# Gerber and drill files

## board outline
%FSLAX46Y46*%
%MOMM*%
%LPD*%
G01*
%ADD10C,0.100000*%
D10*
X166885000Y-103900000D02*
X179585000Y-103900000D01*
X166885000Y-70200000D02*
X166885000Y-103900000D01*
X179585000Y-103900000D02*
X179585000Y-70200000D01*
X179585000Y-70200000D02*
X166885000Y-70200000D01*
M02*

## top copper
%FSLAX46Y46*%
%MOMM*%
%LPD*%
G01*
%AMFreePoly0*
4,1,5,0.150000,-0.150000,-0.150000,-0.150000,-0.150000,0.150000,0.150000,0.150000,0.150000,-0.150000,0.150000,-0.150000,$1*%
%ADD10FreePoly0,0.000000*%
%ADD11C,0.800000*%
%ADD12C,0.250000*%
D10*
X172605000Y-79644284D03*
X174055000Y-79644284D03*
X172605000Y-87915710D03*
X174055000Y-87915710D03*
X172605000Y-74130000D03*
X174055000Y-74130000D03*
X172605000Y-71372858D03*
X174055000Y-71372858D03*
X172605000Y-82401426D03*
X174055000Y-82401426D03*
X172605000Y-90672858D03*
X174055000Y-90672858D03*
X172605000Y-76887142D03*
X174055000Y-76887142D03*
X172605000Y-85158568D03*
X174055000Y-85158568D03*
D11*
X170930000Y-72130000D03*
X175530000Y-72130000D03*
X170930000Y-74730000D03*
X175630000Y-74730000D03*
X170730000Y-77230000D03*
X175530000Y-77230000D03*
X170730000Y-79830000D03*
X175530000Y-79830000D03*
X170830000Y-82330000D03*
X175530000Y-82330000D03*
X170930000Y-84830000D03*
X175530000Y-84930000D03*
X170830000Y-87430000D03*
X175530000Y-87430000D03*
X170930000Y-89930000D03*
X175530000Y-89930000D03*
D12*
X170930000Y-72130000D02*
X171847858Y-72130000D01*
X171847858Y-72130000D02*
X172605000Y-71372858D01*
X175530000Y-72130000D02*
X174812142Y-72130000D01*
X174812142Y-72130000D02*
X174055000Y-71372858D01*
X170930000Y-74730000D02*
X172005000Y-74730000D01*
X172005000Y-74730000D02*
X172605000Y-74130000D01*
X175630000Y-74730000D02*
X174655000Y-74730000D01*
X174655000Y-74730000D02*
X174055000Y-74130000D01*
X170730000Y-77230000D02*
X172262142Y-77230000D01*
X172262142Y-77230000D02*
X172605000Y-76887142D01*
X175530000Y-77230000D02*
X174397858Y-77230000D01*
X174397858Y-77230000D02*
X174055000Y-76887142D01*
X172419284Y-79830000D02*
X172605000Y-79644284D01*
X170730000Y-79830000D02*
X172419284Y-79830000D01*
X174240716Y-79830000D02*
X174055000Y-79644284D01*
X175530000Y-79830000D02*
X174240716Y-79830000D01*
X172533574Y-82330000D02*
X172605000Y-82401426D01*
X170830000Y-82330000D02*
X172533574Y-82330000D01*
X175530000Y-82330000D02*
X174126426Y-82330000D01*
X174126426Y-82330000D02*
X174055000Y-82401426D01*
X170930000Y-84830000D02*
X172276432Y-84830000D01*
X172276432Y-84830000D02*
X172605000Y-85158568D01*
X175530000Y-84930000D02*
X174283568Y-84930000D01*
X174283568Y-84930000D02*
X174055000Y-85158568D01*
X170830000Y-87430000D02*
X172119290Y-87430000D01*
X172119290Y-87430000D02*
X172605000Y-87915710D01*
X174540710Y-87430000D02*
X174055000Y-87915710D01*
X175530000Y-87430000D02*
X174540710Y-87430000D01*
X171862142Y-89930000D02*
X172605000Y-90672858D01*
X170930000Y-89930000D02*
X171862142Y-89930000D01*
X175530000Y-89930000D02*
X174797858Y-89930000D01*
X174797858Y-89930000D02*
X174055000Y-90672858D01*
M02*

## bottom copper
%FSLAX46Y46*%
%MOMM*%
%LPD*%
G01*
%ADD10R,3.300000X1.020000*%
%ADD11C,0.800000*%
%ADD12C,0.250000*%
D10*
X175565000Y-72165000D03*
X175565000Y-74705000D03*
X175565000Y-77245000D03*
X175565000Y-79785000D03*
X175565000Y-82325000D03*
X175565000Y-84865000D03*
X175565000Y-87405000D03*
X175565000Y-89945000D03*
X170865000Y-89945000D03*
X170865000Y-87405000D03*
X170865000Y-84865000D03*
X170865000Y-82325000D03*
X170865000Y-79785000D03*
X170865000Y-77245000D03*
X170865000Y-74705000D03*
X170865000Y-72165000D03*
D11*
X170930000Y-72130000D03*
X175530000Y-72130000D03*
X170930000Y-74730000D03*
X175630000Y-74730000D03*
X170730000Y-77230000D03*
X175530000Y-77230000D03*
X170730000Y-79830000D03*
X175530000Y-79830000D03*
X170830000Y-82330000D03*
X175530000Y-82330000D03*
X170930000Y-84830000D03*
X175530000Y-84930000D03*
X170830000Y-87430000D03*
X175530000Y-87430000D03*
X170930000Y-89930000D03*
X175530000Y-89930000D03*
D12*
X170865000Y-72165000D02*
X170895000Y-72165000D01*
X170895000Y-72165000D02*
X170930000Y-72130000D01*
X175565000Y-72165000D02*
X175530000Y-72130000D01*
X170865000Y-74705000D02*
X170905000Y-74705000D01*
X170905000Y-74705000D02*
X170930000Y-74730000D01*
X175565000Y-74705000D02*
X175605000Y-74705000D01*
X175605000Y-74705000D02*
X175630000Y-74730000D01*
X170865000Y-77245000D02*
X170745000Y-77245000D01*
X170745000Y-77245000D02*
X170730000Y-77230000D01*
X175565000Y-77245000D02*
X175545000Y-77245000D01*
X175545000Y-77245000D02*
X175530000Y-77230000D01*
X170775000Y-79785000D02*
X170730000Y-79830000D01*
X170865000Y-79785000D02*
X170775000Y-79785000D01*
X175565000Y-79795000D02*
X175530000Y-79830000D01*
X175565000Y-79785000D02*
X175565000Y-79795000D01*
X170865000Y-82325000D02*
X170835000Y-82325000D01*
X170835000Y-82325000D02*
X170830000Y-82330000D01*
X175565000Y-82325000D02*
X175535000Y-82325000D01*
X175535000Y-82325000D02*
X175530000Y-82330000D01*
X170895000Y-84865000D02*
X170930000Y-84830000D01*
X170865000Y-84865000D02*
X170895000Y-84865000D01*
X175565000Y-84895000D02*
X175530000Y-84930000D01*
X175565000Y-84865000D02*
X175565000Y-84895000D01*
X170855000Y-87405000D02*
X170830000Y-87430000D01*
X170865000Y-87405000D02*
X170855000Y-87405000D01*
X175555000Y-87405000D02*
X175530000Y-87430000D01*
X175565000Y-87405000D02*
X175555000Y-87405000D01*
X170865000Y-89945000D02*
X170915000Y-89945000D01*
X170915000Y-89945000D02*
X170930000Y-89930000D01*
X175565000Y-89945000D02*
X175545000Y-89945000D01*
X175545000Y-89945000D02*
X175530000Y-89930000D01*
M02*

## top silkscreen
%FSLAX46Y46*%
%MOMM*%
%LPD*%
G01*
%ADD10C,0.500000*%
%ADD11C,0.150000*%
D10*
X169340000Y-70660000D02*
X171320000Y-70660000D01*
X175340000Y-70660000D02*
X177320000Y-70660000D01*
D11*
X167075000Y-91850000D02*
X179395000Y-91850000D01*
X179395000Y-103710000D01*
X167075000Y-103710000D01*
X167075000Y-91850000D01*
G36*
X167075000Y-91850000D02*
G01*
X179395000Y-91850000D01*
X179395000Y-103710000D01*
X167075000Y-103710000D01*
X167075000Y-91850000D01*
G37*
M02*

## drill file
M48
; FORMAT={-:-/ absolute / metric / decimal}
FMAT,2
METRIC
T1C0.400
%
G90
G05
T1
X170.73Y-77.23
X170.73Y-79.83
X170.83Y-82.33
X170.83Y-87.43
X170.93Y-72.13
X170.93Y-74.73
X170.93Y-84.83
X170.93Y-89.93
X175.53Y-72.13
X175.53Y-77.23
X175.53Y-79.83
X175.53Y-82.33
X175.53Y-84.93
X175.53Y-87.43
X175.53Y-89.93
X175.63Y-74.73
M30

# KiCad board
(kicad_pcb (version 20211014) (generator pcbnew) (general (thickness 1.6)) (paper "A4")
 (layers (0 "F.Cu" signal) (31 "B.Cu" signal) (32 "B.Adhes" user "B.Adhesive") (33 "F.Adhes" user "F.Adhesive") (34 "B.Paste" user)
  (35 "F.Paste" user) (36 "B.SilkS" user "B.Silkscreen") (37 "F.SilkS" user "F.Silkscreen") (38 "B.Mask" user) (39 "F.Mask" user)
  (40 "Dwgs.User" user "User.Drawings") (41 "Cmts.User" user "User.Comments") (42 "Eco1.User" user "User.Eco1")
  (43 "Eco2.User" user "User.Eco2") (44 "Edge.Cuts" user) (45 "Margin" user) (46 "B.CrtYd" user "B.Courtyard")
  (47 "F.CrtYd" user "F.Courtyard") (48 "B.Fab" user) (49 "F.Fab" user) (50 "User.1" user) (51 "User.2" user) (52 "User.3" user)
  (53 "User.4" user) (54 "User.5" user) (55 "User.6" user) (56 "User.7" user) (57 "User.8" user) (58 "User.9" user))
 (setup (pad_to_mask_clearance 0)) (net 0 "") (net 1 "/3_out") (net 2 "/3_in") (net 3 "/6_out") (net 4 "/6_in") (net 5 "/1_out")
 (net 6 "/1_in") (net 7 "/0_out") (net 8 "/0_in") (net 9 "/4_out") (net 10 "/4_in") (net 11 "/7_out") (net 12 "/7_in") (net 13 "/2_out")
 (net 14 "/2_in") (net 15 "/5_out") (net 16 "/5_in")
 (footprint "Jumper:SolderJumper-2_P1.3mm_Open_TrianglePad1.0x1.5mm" (layer "F.Cu") (at 173.33 79.644284)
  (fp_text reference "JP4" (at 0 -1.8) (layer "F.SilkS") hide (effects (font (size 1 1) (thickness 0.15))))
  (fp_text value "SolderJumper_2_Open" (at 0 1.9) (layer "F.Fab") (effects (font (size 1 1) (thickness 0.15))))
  (pad "1" smd custom (at -0.725 0) (size 0.3 0.3) (layers "F.Cu" "F.Mask") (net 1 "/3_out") (zone_connect 2)
   (options (clearance outline) (anchor rect)) (primitives))
  (pad "2" smd custom (at 0.725 0) (size 0.3 0.3) (layers "F.Cu" "F.Mask") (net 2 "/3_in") (zone_connect 2)
   (options (clearance outline) (anchor rect)) (primitives)))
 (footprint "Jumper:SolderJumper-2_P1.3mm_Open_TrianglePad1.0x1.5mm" (layer "F.Cu") (at 173.33 87.91571)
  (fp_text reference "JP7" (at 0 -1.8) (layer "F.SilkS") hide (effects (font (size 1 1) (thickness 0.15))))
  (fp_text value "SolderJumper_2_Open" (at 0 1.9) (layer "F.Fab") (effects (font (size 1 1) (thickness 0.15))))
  (pad "1" smd custom (at -0.725 0) (size 0.3 0.3) (layers "F.Cu" "F.Mask") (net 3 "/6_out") (zone_connect 2)
   (options (clearance outline) (anchor rect)) (primitives))
  (pad "2" smd custom (at 0.725 0) (size 0.3 0.3) (layers "F.Cu" "F.Mask") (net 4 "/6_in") (zone_connect 2)
   (options (clearance outline) (anchor rect)) (primitives)))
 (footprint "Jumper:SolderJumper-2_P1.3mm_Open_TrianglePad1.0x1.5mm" (layer "F.Cu") (at 173.33 74.13)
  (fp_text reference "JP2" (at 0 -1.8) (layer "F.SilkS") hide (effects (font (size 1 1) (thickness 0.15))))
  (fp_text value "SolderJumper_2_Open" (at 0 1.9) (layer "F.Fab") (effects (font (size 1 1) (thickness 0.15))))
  (pad "1" smd custom (at -0.725 0) (size 0.3 0.3) (layers "F.Cu" "F.Mask") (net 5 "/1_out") (zone_connect 2)
   (options (clearance outline) (anchor rect)) (primitives))
  (pad "2" smd custom (at 0.725 0) (size 0.3 0.3) (layers "F.Cu" "F.Mask") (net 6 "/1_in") (zone_connect 2)
   (options (clearance outline) (anchor rect)) (primitives)))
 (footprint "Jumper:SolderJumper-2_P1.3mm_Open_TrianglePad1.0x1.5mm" (layer "F.Cu") (at 173.33 71.372858)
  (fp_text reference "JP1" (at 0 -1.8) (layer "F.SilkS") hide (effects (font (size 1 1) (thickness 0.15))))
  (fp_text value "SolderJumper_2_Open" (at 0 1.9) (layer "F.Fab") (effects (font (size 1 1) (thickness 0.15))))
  (pad "1" smd custom (at -0.725 0) (size 0.3 0.3) (layers "F.Cu" "F.Mask") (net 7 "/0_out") (zone_connect 2)
   (options (clearance outline) (anchor rect)) (primitives))
  (pad "2" smd custom (at 0.725 0) (size 0.3 0.3) (layers "F.Cu" "F.Mask") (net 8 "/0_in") (zone_connect 2)
   (options (clearance outline) (anchor rect)) (primitives)))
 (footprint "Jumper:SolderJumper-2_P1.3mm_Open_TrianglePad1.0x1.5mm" (layer "F.Cu") (at 173.33 82.401426)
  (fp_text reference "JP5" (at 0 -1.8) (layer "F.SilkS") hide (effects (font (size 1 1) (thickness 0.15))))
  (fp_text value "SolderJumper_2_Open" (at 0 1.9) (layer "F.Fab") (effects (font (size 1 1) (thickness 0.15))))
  (pad "1" smd custom (at -0.725 0) (size 0.3 0.3) (layers "F.Cu" "F.Mask") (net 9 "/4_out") (zone_connect 2)
   (options (clearance outline) (anchor rect)) (primitives))
  (pad "2" smd custom (at 0.725 0) (size 0.3 0.3) (layers "F.Cu" "F.Mask") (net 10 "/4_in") (zone_connect 2)
   (options (clearance outline) (anchor rect)) (primitives)))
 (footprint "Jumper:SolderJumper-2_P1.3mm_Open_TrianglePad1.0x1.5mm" (layer "F.Cu") (at 173.33 90.672858)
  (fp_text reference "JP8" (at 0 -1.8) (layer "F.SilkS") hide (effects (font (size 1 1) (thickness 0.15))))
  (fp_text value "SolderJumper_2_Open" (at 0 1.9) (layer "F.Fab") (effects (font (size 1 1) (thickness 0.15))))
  (pad "1" smd custom (at -0.725 0) (size 0.3 0.3) (layers "F.Cu" "F.Mask") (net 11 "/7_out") (zone_connect 2)
   (options (clearance outline) (anchor rect)) (primitives))
  (pad "2" smd custom (at 0.725 0) (size 0.3 0.3) (layers "F.Cu" "F.Mask") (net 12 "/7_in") (zone_connect 2)
   (options (clearance outline) (anchor rect)) (primitives)))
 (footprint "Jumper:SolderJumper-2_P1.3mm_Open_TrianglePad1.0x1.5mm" (layer "F.Cu") (at 173.33 76.887142)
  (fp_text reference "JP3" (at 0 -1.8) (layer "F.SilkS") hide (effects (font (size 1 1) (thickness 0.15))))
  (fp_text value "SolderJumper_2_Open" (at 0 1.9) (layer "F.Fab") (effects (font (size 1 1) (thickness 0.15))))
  (pad "1" smd custom (at -0.725 0) (size 0.3 0.3) (layers "F.Cu" "F.Mask") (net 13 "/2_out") (zone_connect 2)
   (options (clearance outline) (anchor rect)) (primitives))
  (pad "2" smd custom (at 0.725 0) (size 0.3 0.3) (layers "F.Cu" "F.Mask") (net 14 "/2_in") (zone_connect 2)
   (options (clearance outline) (anchor rect)) (primitives)))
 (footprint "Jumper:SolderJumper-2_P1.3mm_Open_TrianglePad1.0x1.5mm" (layer "F.Cu") (at 173.33 85.158568)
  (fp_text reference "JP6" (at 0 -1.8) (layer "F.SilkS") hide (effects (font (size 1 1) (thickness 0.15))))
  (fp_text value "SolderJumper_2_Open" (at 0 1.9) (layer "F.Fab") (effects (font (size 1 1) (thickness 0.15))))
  (pad "1" smd custom (at -0.725 0) (size 0.3 0.3) (layers "F.Cu" "F.Mask") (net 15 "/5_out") (zone_connect 2)
   (options (clearance outline) (anchor rect)) (primitives))
  (pad "2" smd custom (at 0.725 0) (size 0.3 0.3) (layers "F.Cu" "F.Mask") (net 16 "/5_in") (zone_connect 2)
   (options (clearance outline) (anchor rect)) (primitives)))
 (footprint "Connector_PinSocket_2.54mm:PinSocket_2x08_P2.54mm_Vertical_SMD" (layer "B.Cu") (at 173.23 81.08 180)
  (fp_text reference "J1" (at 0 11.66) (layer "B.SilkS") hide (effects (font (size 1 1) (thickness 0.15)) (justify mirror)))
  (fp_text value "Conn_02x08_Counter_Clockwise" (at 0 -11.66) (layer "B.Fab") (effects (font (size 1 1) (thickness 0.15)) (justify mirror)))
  (pad "1" smd rect (at -2.335 8.915 180) (size 3.3 1.02) (layers "B.Cu" "B.Paste" "B.Mask") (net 8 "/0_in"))
  (pad "2" smd rect (at -2.335 6.375 180) (size 3.3 1.02) (layers "B.Cu" "B.Paste" "B.Mask") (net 6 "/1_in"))
  (pad "3" smd rect (at -2.335 3.835 180) (size 3.3 1.02) (layers "B.Cu" "B.Paste" "B.Mask") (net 14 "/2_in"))
  (pad "4" smd rect (at -2.335 1.295 180) (size 3.3 1.02) (layers "B.Cu" "B.Paste" "B.Mask") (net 2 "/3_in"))
  (pad "5" smd rect (at -2.335 -1.245 180) (size 3.3 1.02) (layers "B.Cu" "B.Paste" "B.Mask") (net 10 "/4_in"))
  (pad "6" smd rect (at -2.335 -3.785 180) (size 3.3 1.02) (layers "B.Cu" "B.Paste" "B.Mask") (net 16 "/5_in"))
  (pad "7" smd rect (at -2.335 -6.325 180) (size 3.3 1.02) (layers "B.Cu" "B.Paste" "B.Mask") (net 4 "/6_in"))
  (pad "8" smd rect (at -2.335 -8.865 180) (size 3.3 1.02) (layers "B.Cu" "B.Paste" "B.Mask") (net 12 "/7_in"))
  (pad "9" smd rect (at 2.365 -8.865 180) (size 3.3 1.02) (layers "B.Cu" "B.Paste" "B.Mask") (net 11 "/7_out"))
  (pad "10" smd rect (at 2.365 -6.325 180) (size 3.3 1.02) (layers "B.Cu" "B.Paste" "B.Mask") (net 3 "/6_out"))
  (pad "11" smd rect (at 2.365 -3.785 180) (size 3.3 1.02) (layers "B.Cu" "B.Paste" "B.Mask") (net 15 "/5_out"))
  (pad "12" smd rect (at 2.365 -1.245 180) (size 3.3 1.02) (layers "B.Cu" "B.Paste" "B.Mask") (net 9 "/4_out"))
  (pad "13" smd rect (at 2.365 1.295 180) (size 3.3 1.02) (layers "B.Cu" "B.Paste" "B.Mask") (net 1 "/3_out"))
  (pad "14" smd rect (at 2.365 3.835 180) (size 3.3 1.02) (layers "B.Cu" "B.Paste" "B.Mask") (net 13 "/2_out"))
  (pad "15" smd rect (at 2.365 6.375 180) (size 3.3 1.02) (layers "B.Cu" "B.Paste" "B.Mask") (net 5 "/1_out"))
  (pad "16" smd rect (at 2.365 8.915 180) (size 3.3 1.02) (layers "B.Cu" "B.Paste" "B.Mask") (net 7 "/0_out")))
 (gr_line (start 169.34 70.66) (end 171.32 70.66) (layer "F.SilkS") (width 0.5))
 (gr_line (start 175.34 70.66) (end 177.32 70.66) (layer "F.SilkS") (width 0.5))
 (gr_rect (start 167.075 91.85) (end 179.395 103.71) (layer "F.SilkS") (width 0.15) (fill solid))
 (gr_line (start 166.885 103.9) (end 179.585 103.9) (layer "Edge.Cuts") (width 0.1))
 (gr_line (start 166.885 70.2) (end 166.885 103.9) (layer "Edge.Cuts") (width 0.1))
 (gr_line (start 179.585 103.9) (end 179.585 70.2) (layer "Edge.Cuts") (width 0.1))
 (gr_line (start 179.585 70.2) (end 166.885 70.2) (layer "Edge.Cuts") (width 0.1))
 (segment (start 170.93 72.13) (end 171.847858 72.13) (width 0.25) (layer "F.Cu") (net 7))
 (segment (start 171.847858 72.13) (end 172.605 71.372858) (width 0.25) (layer "F.Cu") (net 7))
 (via (at 170.93 72.13) (size 0.8) (drill 0.4) (layers "F.Cu" "B.Cu") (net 7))
 (segment (start 170.865 72.165) (end 170.895 72.165) (width 0.25) (layer "B.Cu") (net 7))
 (segment (start 170.895 72.165) (end 170.93 72.13) (width 0.25) (layer "B.Cu") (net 7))
 (segment (start 175.53 72.13) (end 174.812142 72.13) (width 0.25) (layer "F.Cu") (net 8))
 (segment (start 174.812142 72.13) (end 174.055 71.372858) (width 0.25) (layer "F.Cu") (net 8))
 (via (at 175.53 72.13) (size 0.8) (drill 0.4) (layers "F.Cu" "B.Cu") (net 8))
 (segment (start 175.565 72.165) (end 175.53 72.13) (width 0.25) (layer "B.Cu") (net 8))
 (segment (start 170.93 74.73) (end 172.005 74.73) (width 0.25) (layer "F.Cu") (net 5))
 (segment (start 172.005 74.73) (end 172.605 74.13) (width 0.25) (layer "F.Cu") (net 5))
 (via (at 170.93 74.73) (size 0.8) (drill 0.4) (layers "F.Cu" "B.Cu") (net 5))
 (segment (start 170.865 74.705) (end 170.905 74.705) (width 0.25) (layer "B.Cu") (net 5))
 (segment (start 170.905 74.705) (end 170.93 74.73) (width 0.25) (layer "B.Cu") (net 5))
 (segment (start 175.63 74.73) (end 174.655 74.73) (width 0.25) (layer "F.Cu") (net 6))
 (segment (start 174.655 74.73) (end 174.055 74.13) (width 0.25) (layer "F.Cu") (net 6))
 (via (at 175.63 74.73) (size 0.8) (drill 0.4) (layers "F.Cu" "B.Cu") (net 6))
 (segment (start 175.565 74.705) (end 175.605 74.705) (width 0.25) (layer "B.Cu") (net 6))
 (segment (start 175.605 74.705) (end 175.63 74.73) (width 0.25) (layer "B.Cu") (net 6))
 (segment (start 170.73 77.23) (end 172.262142 77.23) (width 0.25) (layer "F.Cu") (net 13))
 (segment (start 172.262142 77.23) (end 172.605 76.887142) (width 0.25) (layer "F.Cu") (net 13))
 (via (at 170.73 77.23) (size 0.8) (drill 0.4) (layers "F.Cu" "B.Cu") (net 13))
 (segment (start 170.865 77.245) (end 170.745 77.245) (width 0.25) (layer "B.Cu") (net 13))
 (segment (start 170.745 77.245) (end 170.73 77.23) (width 0.25) (layer "B.Cu") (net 13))
 (segment (start 175.53 77.23) (end 174.397858 77.23) (width 0.25) (layer "F.Cu") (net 14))
 (segment (start 174.397858 77.23) (end 174.055 76.887142) (width 0.25) (layer "F.Cu") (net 14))
 (via (at 175.53 77.23) (size 0.8) (drill 0.4) (layers "F.Cu" "B.Cu") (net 14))
 (segment (start 175.565 77.245) (end 175.545 77.245) (width 0.25) (layer "B.Cu") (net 14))
 (segment (start 175.545 77.245) (end 175.53 77.23) (width 0.25) (layer "B.Cu") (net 14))
 (segment (start 172.419284 79.83) (end 172.605 79.644284) (width 0.25) (layer "F.Cu") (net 1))
 (segment (start 170.73 79.83) (end 172.419284 79.83) (width 0.25) (layer "F.Cu") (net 1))
 (via (at 170.73 79.83) (size 0.8) (drill 0.4) (layers "F.Cu" "B.Cu") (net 1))
 (segment (start 170.775 79.785) (end 170.73 79.83) (width 0.25) (layer "B.Cu") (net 1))
 (segment (start 170.865 79.785) (end 170.775 79.785) (width 0.25) (layer "B.Cu") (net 1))
 (segment (start 174.240716 79.83) (end 174.055 79.644284) (width 0.25) (layer "F.Cu") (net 2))
 (segment (start 175.53 79.83) (end 174.240716 79.83) (width 0.25) (layer "F.Cu") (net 2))
 (via (at 175.53 79.83) (size 0.8) (drill 0.4) (layers "F.Cu" "B.Cu") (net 2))
 (segment (start 175.565 79.795) (end 175.53 79.83) (width 0.25) (layer "B.Cu") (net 2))
 (segment (start 175.565 79.785) (end 175.565 79.795) (width 0.25) (layer "B.Cu") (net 2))
 (segment (start 172.533574 82.33) (end 172.605 82.401426) (width 0.25) (layer "F.Cu") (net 9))
 (segment (start 170.83 82.33) (end 172.533574 82.33) (width 0.25) (layer "F.Cu") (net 9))
 (via (at 170.83 82.33) (size 0.8) (drill 0.4) (layers "F.Cu" "B.Cu") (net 9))
 (segment (start 170.865 82.325) (end 170.835 82.325) (width 0.25) (layer "B.Cu") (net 9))
 (segment (start 170.835 82.325) (end 170.83 82.33) (width 0.25) (layer "B.Cu") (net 9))
 (segment (start 175.53 82.33) (end 174.126426 82.33) (width 0.25) (layer "F.Cu") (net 10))
 (segment (start 174.126426 82.33) (end 174.055 82.401426) (width 0.25) (layer "F.Cu") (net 10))
 (via (at 175.53 82.33) (size 0.8) (drill 0.4) (layers "F.Cu" "B.Cu") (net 10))
 (segment (start 175.565 82.325) (end 175.535 82.325) (width 0.25) (layer "B.Cu") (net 10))
 (segment (start 175.535 82.325) (end 175.53 82.33) (width 0.25) (layer "B.Cu") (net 10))
 (segment (start 170.93 84.83) (end 172.276432 84.83) (width 0.25) (layer "F.Cu") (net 15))
 (segment (start 172.276432 84.83) (end 172.605 85.158568) (width 0.25) (layer "F.Cu") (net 15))
 (via (at 170.93 84.83) (size 0.8) (drill 0.4) (layers "F.Cu" "B.Cu") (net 15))
 (segment (start 170.895 84.865) (end 170.93 84.83) (width 0.25) (layer "B.Cu") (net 15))
 (segment (start 170.865 84.865) (end 170.895 84.865) (width 0.25) (layer "B.Cu") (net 15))
 (segment (start 175.53 84.93) (end 174.283568 84.93) (width 0.25) (layer "F.Cu") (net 16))
 (segment (start 174.283568 84.93) (end 174.055 85.158568) (width 0.25) (layer "F.Cu") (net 16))
 (via (at 175.53 84.93) (size 0.8) (drill 0.4) (layers "F.Cu" "B.Cu") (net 16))
 (segment (start 175.565 84.895) (end 175.53 84.93) (width 0.25) (layer "B.Cu") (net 16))
 (segment (start 175.565 84.865) (end 175.565 84.895) (width 0.25) (layer "B.Cu") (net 16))
 (segment (start 170.83 87.43) (end 172.11929 87.43) (width 0.25) (layer "F.Cu") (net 3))
 (segment (start 172.11929 87.43) (end 172.605 87.91571) (width 0.25) (layer "F.Cu") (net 3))
 (via (at 170.83 87.43) (size 0.8) (drill 0.4) (layers "F.Cu" "B.Cu") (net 3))
 (segment (start 170.855 87.405) (end 170.83 87.43) (width 0.25) (layer "B.Cu") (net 3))
 (segment (start 170.865 87.405) (end 170.855 87.405) (width 0.25) (layer "B.Cu") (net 3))
 (segment (start 174.54071 87.43) (end 174.055 87.91571) (width 0.25) (layer "F.Cu") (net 4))
 (segment (start 175.53 87.43) (end 174.54071 87.43) (width 0.25) (layer "F.Cu") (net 4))
 (via (at 175.53 87.43) (size 0.8) (drill 0.4) (layers "F.Cu" "B.Cu") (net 4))
 (segment (start 175.555 87.405) (end 175.53 87.43) (width 0.25) (layer "B.Cu") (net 4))
 (segment (start 175.565 87.405) (end 175.555 87.405) (width 0.25) (layer "B.Cu") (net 4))
 (segment (start 171.862142 89.93) (end 172.605 90.672858) (width 0.25) (layer "F.Cu") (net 11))
 (segment (start 170.93 89.93) (end 171.862142 89.93) (width 0.25) (layer "F.Cu") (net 11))
 (via (at 170.93 89.93) (size 0.8) (drill 0.4) (layers "F.Cu" "B.Cu") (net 11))
 (segment (start 170.865 89.945) (end 170.915 89.945) (width 0.25) (layer "B.Cu") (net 11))
 (segment (start 170.915 89.945) (end 170.93 89.93) (width 0.25) (layer "B.Cu") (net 11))
 (segment (start 175.53 89.93) (end 174.797858 89.93) (width 0.25) (layer "F.Cu") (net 12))
 (segment (start 174.797858 89.93) (end 174.055 90.672858) (width 0.25) (layer "F.Cu") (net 12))
 (via (at 175.53 89.93) (size 0.8) (drill 0.4) (layers "F.Cu" "B.Cu") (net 12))
 (segment (start 175.565 89.945) (end 175.545 89.945) (width 0.25) (layer "B.Cu") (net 12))
 (segment (start 175.545 89.945) (end 175.53 89.93) (width 0.25) (layer "B.Cu") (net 12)))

